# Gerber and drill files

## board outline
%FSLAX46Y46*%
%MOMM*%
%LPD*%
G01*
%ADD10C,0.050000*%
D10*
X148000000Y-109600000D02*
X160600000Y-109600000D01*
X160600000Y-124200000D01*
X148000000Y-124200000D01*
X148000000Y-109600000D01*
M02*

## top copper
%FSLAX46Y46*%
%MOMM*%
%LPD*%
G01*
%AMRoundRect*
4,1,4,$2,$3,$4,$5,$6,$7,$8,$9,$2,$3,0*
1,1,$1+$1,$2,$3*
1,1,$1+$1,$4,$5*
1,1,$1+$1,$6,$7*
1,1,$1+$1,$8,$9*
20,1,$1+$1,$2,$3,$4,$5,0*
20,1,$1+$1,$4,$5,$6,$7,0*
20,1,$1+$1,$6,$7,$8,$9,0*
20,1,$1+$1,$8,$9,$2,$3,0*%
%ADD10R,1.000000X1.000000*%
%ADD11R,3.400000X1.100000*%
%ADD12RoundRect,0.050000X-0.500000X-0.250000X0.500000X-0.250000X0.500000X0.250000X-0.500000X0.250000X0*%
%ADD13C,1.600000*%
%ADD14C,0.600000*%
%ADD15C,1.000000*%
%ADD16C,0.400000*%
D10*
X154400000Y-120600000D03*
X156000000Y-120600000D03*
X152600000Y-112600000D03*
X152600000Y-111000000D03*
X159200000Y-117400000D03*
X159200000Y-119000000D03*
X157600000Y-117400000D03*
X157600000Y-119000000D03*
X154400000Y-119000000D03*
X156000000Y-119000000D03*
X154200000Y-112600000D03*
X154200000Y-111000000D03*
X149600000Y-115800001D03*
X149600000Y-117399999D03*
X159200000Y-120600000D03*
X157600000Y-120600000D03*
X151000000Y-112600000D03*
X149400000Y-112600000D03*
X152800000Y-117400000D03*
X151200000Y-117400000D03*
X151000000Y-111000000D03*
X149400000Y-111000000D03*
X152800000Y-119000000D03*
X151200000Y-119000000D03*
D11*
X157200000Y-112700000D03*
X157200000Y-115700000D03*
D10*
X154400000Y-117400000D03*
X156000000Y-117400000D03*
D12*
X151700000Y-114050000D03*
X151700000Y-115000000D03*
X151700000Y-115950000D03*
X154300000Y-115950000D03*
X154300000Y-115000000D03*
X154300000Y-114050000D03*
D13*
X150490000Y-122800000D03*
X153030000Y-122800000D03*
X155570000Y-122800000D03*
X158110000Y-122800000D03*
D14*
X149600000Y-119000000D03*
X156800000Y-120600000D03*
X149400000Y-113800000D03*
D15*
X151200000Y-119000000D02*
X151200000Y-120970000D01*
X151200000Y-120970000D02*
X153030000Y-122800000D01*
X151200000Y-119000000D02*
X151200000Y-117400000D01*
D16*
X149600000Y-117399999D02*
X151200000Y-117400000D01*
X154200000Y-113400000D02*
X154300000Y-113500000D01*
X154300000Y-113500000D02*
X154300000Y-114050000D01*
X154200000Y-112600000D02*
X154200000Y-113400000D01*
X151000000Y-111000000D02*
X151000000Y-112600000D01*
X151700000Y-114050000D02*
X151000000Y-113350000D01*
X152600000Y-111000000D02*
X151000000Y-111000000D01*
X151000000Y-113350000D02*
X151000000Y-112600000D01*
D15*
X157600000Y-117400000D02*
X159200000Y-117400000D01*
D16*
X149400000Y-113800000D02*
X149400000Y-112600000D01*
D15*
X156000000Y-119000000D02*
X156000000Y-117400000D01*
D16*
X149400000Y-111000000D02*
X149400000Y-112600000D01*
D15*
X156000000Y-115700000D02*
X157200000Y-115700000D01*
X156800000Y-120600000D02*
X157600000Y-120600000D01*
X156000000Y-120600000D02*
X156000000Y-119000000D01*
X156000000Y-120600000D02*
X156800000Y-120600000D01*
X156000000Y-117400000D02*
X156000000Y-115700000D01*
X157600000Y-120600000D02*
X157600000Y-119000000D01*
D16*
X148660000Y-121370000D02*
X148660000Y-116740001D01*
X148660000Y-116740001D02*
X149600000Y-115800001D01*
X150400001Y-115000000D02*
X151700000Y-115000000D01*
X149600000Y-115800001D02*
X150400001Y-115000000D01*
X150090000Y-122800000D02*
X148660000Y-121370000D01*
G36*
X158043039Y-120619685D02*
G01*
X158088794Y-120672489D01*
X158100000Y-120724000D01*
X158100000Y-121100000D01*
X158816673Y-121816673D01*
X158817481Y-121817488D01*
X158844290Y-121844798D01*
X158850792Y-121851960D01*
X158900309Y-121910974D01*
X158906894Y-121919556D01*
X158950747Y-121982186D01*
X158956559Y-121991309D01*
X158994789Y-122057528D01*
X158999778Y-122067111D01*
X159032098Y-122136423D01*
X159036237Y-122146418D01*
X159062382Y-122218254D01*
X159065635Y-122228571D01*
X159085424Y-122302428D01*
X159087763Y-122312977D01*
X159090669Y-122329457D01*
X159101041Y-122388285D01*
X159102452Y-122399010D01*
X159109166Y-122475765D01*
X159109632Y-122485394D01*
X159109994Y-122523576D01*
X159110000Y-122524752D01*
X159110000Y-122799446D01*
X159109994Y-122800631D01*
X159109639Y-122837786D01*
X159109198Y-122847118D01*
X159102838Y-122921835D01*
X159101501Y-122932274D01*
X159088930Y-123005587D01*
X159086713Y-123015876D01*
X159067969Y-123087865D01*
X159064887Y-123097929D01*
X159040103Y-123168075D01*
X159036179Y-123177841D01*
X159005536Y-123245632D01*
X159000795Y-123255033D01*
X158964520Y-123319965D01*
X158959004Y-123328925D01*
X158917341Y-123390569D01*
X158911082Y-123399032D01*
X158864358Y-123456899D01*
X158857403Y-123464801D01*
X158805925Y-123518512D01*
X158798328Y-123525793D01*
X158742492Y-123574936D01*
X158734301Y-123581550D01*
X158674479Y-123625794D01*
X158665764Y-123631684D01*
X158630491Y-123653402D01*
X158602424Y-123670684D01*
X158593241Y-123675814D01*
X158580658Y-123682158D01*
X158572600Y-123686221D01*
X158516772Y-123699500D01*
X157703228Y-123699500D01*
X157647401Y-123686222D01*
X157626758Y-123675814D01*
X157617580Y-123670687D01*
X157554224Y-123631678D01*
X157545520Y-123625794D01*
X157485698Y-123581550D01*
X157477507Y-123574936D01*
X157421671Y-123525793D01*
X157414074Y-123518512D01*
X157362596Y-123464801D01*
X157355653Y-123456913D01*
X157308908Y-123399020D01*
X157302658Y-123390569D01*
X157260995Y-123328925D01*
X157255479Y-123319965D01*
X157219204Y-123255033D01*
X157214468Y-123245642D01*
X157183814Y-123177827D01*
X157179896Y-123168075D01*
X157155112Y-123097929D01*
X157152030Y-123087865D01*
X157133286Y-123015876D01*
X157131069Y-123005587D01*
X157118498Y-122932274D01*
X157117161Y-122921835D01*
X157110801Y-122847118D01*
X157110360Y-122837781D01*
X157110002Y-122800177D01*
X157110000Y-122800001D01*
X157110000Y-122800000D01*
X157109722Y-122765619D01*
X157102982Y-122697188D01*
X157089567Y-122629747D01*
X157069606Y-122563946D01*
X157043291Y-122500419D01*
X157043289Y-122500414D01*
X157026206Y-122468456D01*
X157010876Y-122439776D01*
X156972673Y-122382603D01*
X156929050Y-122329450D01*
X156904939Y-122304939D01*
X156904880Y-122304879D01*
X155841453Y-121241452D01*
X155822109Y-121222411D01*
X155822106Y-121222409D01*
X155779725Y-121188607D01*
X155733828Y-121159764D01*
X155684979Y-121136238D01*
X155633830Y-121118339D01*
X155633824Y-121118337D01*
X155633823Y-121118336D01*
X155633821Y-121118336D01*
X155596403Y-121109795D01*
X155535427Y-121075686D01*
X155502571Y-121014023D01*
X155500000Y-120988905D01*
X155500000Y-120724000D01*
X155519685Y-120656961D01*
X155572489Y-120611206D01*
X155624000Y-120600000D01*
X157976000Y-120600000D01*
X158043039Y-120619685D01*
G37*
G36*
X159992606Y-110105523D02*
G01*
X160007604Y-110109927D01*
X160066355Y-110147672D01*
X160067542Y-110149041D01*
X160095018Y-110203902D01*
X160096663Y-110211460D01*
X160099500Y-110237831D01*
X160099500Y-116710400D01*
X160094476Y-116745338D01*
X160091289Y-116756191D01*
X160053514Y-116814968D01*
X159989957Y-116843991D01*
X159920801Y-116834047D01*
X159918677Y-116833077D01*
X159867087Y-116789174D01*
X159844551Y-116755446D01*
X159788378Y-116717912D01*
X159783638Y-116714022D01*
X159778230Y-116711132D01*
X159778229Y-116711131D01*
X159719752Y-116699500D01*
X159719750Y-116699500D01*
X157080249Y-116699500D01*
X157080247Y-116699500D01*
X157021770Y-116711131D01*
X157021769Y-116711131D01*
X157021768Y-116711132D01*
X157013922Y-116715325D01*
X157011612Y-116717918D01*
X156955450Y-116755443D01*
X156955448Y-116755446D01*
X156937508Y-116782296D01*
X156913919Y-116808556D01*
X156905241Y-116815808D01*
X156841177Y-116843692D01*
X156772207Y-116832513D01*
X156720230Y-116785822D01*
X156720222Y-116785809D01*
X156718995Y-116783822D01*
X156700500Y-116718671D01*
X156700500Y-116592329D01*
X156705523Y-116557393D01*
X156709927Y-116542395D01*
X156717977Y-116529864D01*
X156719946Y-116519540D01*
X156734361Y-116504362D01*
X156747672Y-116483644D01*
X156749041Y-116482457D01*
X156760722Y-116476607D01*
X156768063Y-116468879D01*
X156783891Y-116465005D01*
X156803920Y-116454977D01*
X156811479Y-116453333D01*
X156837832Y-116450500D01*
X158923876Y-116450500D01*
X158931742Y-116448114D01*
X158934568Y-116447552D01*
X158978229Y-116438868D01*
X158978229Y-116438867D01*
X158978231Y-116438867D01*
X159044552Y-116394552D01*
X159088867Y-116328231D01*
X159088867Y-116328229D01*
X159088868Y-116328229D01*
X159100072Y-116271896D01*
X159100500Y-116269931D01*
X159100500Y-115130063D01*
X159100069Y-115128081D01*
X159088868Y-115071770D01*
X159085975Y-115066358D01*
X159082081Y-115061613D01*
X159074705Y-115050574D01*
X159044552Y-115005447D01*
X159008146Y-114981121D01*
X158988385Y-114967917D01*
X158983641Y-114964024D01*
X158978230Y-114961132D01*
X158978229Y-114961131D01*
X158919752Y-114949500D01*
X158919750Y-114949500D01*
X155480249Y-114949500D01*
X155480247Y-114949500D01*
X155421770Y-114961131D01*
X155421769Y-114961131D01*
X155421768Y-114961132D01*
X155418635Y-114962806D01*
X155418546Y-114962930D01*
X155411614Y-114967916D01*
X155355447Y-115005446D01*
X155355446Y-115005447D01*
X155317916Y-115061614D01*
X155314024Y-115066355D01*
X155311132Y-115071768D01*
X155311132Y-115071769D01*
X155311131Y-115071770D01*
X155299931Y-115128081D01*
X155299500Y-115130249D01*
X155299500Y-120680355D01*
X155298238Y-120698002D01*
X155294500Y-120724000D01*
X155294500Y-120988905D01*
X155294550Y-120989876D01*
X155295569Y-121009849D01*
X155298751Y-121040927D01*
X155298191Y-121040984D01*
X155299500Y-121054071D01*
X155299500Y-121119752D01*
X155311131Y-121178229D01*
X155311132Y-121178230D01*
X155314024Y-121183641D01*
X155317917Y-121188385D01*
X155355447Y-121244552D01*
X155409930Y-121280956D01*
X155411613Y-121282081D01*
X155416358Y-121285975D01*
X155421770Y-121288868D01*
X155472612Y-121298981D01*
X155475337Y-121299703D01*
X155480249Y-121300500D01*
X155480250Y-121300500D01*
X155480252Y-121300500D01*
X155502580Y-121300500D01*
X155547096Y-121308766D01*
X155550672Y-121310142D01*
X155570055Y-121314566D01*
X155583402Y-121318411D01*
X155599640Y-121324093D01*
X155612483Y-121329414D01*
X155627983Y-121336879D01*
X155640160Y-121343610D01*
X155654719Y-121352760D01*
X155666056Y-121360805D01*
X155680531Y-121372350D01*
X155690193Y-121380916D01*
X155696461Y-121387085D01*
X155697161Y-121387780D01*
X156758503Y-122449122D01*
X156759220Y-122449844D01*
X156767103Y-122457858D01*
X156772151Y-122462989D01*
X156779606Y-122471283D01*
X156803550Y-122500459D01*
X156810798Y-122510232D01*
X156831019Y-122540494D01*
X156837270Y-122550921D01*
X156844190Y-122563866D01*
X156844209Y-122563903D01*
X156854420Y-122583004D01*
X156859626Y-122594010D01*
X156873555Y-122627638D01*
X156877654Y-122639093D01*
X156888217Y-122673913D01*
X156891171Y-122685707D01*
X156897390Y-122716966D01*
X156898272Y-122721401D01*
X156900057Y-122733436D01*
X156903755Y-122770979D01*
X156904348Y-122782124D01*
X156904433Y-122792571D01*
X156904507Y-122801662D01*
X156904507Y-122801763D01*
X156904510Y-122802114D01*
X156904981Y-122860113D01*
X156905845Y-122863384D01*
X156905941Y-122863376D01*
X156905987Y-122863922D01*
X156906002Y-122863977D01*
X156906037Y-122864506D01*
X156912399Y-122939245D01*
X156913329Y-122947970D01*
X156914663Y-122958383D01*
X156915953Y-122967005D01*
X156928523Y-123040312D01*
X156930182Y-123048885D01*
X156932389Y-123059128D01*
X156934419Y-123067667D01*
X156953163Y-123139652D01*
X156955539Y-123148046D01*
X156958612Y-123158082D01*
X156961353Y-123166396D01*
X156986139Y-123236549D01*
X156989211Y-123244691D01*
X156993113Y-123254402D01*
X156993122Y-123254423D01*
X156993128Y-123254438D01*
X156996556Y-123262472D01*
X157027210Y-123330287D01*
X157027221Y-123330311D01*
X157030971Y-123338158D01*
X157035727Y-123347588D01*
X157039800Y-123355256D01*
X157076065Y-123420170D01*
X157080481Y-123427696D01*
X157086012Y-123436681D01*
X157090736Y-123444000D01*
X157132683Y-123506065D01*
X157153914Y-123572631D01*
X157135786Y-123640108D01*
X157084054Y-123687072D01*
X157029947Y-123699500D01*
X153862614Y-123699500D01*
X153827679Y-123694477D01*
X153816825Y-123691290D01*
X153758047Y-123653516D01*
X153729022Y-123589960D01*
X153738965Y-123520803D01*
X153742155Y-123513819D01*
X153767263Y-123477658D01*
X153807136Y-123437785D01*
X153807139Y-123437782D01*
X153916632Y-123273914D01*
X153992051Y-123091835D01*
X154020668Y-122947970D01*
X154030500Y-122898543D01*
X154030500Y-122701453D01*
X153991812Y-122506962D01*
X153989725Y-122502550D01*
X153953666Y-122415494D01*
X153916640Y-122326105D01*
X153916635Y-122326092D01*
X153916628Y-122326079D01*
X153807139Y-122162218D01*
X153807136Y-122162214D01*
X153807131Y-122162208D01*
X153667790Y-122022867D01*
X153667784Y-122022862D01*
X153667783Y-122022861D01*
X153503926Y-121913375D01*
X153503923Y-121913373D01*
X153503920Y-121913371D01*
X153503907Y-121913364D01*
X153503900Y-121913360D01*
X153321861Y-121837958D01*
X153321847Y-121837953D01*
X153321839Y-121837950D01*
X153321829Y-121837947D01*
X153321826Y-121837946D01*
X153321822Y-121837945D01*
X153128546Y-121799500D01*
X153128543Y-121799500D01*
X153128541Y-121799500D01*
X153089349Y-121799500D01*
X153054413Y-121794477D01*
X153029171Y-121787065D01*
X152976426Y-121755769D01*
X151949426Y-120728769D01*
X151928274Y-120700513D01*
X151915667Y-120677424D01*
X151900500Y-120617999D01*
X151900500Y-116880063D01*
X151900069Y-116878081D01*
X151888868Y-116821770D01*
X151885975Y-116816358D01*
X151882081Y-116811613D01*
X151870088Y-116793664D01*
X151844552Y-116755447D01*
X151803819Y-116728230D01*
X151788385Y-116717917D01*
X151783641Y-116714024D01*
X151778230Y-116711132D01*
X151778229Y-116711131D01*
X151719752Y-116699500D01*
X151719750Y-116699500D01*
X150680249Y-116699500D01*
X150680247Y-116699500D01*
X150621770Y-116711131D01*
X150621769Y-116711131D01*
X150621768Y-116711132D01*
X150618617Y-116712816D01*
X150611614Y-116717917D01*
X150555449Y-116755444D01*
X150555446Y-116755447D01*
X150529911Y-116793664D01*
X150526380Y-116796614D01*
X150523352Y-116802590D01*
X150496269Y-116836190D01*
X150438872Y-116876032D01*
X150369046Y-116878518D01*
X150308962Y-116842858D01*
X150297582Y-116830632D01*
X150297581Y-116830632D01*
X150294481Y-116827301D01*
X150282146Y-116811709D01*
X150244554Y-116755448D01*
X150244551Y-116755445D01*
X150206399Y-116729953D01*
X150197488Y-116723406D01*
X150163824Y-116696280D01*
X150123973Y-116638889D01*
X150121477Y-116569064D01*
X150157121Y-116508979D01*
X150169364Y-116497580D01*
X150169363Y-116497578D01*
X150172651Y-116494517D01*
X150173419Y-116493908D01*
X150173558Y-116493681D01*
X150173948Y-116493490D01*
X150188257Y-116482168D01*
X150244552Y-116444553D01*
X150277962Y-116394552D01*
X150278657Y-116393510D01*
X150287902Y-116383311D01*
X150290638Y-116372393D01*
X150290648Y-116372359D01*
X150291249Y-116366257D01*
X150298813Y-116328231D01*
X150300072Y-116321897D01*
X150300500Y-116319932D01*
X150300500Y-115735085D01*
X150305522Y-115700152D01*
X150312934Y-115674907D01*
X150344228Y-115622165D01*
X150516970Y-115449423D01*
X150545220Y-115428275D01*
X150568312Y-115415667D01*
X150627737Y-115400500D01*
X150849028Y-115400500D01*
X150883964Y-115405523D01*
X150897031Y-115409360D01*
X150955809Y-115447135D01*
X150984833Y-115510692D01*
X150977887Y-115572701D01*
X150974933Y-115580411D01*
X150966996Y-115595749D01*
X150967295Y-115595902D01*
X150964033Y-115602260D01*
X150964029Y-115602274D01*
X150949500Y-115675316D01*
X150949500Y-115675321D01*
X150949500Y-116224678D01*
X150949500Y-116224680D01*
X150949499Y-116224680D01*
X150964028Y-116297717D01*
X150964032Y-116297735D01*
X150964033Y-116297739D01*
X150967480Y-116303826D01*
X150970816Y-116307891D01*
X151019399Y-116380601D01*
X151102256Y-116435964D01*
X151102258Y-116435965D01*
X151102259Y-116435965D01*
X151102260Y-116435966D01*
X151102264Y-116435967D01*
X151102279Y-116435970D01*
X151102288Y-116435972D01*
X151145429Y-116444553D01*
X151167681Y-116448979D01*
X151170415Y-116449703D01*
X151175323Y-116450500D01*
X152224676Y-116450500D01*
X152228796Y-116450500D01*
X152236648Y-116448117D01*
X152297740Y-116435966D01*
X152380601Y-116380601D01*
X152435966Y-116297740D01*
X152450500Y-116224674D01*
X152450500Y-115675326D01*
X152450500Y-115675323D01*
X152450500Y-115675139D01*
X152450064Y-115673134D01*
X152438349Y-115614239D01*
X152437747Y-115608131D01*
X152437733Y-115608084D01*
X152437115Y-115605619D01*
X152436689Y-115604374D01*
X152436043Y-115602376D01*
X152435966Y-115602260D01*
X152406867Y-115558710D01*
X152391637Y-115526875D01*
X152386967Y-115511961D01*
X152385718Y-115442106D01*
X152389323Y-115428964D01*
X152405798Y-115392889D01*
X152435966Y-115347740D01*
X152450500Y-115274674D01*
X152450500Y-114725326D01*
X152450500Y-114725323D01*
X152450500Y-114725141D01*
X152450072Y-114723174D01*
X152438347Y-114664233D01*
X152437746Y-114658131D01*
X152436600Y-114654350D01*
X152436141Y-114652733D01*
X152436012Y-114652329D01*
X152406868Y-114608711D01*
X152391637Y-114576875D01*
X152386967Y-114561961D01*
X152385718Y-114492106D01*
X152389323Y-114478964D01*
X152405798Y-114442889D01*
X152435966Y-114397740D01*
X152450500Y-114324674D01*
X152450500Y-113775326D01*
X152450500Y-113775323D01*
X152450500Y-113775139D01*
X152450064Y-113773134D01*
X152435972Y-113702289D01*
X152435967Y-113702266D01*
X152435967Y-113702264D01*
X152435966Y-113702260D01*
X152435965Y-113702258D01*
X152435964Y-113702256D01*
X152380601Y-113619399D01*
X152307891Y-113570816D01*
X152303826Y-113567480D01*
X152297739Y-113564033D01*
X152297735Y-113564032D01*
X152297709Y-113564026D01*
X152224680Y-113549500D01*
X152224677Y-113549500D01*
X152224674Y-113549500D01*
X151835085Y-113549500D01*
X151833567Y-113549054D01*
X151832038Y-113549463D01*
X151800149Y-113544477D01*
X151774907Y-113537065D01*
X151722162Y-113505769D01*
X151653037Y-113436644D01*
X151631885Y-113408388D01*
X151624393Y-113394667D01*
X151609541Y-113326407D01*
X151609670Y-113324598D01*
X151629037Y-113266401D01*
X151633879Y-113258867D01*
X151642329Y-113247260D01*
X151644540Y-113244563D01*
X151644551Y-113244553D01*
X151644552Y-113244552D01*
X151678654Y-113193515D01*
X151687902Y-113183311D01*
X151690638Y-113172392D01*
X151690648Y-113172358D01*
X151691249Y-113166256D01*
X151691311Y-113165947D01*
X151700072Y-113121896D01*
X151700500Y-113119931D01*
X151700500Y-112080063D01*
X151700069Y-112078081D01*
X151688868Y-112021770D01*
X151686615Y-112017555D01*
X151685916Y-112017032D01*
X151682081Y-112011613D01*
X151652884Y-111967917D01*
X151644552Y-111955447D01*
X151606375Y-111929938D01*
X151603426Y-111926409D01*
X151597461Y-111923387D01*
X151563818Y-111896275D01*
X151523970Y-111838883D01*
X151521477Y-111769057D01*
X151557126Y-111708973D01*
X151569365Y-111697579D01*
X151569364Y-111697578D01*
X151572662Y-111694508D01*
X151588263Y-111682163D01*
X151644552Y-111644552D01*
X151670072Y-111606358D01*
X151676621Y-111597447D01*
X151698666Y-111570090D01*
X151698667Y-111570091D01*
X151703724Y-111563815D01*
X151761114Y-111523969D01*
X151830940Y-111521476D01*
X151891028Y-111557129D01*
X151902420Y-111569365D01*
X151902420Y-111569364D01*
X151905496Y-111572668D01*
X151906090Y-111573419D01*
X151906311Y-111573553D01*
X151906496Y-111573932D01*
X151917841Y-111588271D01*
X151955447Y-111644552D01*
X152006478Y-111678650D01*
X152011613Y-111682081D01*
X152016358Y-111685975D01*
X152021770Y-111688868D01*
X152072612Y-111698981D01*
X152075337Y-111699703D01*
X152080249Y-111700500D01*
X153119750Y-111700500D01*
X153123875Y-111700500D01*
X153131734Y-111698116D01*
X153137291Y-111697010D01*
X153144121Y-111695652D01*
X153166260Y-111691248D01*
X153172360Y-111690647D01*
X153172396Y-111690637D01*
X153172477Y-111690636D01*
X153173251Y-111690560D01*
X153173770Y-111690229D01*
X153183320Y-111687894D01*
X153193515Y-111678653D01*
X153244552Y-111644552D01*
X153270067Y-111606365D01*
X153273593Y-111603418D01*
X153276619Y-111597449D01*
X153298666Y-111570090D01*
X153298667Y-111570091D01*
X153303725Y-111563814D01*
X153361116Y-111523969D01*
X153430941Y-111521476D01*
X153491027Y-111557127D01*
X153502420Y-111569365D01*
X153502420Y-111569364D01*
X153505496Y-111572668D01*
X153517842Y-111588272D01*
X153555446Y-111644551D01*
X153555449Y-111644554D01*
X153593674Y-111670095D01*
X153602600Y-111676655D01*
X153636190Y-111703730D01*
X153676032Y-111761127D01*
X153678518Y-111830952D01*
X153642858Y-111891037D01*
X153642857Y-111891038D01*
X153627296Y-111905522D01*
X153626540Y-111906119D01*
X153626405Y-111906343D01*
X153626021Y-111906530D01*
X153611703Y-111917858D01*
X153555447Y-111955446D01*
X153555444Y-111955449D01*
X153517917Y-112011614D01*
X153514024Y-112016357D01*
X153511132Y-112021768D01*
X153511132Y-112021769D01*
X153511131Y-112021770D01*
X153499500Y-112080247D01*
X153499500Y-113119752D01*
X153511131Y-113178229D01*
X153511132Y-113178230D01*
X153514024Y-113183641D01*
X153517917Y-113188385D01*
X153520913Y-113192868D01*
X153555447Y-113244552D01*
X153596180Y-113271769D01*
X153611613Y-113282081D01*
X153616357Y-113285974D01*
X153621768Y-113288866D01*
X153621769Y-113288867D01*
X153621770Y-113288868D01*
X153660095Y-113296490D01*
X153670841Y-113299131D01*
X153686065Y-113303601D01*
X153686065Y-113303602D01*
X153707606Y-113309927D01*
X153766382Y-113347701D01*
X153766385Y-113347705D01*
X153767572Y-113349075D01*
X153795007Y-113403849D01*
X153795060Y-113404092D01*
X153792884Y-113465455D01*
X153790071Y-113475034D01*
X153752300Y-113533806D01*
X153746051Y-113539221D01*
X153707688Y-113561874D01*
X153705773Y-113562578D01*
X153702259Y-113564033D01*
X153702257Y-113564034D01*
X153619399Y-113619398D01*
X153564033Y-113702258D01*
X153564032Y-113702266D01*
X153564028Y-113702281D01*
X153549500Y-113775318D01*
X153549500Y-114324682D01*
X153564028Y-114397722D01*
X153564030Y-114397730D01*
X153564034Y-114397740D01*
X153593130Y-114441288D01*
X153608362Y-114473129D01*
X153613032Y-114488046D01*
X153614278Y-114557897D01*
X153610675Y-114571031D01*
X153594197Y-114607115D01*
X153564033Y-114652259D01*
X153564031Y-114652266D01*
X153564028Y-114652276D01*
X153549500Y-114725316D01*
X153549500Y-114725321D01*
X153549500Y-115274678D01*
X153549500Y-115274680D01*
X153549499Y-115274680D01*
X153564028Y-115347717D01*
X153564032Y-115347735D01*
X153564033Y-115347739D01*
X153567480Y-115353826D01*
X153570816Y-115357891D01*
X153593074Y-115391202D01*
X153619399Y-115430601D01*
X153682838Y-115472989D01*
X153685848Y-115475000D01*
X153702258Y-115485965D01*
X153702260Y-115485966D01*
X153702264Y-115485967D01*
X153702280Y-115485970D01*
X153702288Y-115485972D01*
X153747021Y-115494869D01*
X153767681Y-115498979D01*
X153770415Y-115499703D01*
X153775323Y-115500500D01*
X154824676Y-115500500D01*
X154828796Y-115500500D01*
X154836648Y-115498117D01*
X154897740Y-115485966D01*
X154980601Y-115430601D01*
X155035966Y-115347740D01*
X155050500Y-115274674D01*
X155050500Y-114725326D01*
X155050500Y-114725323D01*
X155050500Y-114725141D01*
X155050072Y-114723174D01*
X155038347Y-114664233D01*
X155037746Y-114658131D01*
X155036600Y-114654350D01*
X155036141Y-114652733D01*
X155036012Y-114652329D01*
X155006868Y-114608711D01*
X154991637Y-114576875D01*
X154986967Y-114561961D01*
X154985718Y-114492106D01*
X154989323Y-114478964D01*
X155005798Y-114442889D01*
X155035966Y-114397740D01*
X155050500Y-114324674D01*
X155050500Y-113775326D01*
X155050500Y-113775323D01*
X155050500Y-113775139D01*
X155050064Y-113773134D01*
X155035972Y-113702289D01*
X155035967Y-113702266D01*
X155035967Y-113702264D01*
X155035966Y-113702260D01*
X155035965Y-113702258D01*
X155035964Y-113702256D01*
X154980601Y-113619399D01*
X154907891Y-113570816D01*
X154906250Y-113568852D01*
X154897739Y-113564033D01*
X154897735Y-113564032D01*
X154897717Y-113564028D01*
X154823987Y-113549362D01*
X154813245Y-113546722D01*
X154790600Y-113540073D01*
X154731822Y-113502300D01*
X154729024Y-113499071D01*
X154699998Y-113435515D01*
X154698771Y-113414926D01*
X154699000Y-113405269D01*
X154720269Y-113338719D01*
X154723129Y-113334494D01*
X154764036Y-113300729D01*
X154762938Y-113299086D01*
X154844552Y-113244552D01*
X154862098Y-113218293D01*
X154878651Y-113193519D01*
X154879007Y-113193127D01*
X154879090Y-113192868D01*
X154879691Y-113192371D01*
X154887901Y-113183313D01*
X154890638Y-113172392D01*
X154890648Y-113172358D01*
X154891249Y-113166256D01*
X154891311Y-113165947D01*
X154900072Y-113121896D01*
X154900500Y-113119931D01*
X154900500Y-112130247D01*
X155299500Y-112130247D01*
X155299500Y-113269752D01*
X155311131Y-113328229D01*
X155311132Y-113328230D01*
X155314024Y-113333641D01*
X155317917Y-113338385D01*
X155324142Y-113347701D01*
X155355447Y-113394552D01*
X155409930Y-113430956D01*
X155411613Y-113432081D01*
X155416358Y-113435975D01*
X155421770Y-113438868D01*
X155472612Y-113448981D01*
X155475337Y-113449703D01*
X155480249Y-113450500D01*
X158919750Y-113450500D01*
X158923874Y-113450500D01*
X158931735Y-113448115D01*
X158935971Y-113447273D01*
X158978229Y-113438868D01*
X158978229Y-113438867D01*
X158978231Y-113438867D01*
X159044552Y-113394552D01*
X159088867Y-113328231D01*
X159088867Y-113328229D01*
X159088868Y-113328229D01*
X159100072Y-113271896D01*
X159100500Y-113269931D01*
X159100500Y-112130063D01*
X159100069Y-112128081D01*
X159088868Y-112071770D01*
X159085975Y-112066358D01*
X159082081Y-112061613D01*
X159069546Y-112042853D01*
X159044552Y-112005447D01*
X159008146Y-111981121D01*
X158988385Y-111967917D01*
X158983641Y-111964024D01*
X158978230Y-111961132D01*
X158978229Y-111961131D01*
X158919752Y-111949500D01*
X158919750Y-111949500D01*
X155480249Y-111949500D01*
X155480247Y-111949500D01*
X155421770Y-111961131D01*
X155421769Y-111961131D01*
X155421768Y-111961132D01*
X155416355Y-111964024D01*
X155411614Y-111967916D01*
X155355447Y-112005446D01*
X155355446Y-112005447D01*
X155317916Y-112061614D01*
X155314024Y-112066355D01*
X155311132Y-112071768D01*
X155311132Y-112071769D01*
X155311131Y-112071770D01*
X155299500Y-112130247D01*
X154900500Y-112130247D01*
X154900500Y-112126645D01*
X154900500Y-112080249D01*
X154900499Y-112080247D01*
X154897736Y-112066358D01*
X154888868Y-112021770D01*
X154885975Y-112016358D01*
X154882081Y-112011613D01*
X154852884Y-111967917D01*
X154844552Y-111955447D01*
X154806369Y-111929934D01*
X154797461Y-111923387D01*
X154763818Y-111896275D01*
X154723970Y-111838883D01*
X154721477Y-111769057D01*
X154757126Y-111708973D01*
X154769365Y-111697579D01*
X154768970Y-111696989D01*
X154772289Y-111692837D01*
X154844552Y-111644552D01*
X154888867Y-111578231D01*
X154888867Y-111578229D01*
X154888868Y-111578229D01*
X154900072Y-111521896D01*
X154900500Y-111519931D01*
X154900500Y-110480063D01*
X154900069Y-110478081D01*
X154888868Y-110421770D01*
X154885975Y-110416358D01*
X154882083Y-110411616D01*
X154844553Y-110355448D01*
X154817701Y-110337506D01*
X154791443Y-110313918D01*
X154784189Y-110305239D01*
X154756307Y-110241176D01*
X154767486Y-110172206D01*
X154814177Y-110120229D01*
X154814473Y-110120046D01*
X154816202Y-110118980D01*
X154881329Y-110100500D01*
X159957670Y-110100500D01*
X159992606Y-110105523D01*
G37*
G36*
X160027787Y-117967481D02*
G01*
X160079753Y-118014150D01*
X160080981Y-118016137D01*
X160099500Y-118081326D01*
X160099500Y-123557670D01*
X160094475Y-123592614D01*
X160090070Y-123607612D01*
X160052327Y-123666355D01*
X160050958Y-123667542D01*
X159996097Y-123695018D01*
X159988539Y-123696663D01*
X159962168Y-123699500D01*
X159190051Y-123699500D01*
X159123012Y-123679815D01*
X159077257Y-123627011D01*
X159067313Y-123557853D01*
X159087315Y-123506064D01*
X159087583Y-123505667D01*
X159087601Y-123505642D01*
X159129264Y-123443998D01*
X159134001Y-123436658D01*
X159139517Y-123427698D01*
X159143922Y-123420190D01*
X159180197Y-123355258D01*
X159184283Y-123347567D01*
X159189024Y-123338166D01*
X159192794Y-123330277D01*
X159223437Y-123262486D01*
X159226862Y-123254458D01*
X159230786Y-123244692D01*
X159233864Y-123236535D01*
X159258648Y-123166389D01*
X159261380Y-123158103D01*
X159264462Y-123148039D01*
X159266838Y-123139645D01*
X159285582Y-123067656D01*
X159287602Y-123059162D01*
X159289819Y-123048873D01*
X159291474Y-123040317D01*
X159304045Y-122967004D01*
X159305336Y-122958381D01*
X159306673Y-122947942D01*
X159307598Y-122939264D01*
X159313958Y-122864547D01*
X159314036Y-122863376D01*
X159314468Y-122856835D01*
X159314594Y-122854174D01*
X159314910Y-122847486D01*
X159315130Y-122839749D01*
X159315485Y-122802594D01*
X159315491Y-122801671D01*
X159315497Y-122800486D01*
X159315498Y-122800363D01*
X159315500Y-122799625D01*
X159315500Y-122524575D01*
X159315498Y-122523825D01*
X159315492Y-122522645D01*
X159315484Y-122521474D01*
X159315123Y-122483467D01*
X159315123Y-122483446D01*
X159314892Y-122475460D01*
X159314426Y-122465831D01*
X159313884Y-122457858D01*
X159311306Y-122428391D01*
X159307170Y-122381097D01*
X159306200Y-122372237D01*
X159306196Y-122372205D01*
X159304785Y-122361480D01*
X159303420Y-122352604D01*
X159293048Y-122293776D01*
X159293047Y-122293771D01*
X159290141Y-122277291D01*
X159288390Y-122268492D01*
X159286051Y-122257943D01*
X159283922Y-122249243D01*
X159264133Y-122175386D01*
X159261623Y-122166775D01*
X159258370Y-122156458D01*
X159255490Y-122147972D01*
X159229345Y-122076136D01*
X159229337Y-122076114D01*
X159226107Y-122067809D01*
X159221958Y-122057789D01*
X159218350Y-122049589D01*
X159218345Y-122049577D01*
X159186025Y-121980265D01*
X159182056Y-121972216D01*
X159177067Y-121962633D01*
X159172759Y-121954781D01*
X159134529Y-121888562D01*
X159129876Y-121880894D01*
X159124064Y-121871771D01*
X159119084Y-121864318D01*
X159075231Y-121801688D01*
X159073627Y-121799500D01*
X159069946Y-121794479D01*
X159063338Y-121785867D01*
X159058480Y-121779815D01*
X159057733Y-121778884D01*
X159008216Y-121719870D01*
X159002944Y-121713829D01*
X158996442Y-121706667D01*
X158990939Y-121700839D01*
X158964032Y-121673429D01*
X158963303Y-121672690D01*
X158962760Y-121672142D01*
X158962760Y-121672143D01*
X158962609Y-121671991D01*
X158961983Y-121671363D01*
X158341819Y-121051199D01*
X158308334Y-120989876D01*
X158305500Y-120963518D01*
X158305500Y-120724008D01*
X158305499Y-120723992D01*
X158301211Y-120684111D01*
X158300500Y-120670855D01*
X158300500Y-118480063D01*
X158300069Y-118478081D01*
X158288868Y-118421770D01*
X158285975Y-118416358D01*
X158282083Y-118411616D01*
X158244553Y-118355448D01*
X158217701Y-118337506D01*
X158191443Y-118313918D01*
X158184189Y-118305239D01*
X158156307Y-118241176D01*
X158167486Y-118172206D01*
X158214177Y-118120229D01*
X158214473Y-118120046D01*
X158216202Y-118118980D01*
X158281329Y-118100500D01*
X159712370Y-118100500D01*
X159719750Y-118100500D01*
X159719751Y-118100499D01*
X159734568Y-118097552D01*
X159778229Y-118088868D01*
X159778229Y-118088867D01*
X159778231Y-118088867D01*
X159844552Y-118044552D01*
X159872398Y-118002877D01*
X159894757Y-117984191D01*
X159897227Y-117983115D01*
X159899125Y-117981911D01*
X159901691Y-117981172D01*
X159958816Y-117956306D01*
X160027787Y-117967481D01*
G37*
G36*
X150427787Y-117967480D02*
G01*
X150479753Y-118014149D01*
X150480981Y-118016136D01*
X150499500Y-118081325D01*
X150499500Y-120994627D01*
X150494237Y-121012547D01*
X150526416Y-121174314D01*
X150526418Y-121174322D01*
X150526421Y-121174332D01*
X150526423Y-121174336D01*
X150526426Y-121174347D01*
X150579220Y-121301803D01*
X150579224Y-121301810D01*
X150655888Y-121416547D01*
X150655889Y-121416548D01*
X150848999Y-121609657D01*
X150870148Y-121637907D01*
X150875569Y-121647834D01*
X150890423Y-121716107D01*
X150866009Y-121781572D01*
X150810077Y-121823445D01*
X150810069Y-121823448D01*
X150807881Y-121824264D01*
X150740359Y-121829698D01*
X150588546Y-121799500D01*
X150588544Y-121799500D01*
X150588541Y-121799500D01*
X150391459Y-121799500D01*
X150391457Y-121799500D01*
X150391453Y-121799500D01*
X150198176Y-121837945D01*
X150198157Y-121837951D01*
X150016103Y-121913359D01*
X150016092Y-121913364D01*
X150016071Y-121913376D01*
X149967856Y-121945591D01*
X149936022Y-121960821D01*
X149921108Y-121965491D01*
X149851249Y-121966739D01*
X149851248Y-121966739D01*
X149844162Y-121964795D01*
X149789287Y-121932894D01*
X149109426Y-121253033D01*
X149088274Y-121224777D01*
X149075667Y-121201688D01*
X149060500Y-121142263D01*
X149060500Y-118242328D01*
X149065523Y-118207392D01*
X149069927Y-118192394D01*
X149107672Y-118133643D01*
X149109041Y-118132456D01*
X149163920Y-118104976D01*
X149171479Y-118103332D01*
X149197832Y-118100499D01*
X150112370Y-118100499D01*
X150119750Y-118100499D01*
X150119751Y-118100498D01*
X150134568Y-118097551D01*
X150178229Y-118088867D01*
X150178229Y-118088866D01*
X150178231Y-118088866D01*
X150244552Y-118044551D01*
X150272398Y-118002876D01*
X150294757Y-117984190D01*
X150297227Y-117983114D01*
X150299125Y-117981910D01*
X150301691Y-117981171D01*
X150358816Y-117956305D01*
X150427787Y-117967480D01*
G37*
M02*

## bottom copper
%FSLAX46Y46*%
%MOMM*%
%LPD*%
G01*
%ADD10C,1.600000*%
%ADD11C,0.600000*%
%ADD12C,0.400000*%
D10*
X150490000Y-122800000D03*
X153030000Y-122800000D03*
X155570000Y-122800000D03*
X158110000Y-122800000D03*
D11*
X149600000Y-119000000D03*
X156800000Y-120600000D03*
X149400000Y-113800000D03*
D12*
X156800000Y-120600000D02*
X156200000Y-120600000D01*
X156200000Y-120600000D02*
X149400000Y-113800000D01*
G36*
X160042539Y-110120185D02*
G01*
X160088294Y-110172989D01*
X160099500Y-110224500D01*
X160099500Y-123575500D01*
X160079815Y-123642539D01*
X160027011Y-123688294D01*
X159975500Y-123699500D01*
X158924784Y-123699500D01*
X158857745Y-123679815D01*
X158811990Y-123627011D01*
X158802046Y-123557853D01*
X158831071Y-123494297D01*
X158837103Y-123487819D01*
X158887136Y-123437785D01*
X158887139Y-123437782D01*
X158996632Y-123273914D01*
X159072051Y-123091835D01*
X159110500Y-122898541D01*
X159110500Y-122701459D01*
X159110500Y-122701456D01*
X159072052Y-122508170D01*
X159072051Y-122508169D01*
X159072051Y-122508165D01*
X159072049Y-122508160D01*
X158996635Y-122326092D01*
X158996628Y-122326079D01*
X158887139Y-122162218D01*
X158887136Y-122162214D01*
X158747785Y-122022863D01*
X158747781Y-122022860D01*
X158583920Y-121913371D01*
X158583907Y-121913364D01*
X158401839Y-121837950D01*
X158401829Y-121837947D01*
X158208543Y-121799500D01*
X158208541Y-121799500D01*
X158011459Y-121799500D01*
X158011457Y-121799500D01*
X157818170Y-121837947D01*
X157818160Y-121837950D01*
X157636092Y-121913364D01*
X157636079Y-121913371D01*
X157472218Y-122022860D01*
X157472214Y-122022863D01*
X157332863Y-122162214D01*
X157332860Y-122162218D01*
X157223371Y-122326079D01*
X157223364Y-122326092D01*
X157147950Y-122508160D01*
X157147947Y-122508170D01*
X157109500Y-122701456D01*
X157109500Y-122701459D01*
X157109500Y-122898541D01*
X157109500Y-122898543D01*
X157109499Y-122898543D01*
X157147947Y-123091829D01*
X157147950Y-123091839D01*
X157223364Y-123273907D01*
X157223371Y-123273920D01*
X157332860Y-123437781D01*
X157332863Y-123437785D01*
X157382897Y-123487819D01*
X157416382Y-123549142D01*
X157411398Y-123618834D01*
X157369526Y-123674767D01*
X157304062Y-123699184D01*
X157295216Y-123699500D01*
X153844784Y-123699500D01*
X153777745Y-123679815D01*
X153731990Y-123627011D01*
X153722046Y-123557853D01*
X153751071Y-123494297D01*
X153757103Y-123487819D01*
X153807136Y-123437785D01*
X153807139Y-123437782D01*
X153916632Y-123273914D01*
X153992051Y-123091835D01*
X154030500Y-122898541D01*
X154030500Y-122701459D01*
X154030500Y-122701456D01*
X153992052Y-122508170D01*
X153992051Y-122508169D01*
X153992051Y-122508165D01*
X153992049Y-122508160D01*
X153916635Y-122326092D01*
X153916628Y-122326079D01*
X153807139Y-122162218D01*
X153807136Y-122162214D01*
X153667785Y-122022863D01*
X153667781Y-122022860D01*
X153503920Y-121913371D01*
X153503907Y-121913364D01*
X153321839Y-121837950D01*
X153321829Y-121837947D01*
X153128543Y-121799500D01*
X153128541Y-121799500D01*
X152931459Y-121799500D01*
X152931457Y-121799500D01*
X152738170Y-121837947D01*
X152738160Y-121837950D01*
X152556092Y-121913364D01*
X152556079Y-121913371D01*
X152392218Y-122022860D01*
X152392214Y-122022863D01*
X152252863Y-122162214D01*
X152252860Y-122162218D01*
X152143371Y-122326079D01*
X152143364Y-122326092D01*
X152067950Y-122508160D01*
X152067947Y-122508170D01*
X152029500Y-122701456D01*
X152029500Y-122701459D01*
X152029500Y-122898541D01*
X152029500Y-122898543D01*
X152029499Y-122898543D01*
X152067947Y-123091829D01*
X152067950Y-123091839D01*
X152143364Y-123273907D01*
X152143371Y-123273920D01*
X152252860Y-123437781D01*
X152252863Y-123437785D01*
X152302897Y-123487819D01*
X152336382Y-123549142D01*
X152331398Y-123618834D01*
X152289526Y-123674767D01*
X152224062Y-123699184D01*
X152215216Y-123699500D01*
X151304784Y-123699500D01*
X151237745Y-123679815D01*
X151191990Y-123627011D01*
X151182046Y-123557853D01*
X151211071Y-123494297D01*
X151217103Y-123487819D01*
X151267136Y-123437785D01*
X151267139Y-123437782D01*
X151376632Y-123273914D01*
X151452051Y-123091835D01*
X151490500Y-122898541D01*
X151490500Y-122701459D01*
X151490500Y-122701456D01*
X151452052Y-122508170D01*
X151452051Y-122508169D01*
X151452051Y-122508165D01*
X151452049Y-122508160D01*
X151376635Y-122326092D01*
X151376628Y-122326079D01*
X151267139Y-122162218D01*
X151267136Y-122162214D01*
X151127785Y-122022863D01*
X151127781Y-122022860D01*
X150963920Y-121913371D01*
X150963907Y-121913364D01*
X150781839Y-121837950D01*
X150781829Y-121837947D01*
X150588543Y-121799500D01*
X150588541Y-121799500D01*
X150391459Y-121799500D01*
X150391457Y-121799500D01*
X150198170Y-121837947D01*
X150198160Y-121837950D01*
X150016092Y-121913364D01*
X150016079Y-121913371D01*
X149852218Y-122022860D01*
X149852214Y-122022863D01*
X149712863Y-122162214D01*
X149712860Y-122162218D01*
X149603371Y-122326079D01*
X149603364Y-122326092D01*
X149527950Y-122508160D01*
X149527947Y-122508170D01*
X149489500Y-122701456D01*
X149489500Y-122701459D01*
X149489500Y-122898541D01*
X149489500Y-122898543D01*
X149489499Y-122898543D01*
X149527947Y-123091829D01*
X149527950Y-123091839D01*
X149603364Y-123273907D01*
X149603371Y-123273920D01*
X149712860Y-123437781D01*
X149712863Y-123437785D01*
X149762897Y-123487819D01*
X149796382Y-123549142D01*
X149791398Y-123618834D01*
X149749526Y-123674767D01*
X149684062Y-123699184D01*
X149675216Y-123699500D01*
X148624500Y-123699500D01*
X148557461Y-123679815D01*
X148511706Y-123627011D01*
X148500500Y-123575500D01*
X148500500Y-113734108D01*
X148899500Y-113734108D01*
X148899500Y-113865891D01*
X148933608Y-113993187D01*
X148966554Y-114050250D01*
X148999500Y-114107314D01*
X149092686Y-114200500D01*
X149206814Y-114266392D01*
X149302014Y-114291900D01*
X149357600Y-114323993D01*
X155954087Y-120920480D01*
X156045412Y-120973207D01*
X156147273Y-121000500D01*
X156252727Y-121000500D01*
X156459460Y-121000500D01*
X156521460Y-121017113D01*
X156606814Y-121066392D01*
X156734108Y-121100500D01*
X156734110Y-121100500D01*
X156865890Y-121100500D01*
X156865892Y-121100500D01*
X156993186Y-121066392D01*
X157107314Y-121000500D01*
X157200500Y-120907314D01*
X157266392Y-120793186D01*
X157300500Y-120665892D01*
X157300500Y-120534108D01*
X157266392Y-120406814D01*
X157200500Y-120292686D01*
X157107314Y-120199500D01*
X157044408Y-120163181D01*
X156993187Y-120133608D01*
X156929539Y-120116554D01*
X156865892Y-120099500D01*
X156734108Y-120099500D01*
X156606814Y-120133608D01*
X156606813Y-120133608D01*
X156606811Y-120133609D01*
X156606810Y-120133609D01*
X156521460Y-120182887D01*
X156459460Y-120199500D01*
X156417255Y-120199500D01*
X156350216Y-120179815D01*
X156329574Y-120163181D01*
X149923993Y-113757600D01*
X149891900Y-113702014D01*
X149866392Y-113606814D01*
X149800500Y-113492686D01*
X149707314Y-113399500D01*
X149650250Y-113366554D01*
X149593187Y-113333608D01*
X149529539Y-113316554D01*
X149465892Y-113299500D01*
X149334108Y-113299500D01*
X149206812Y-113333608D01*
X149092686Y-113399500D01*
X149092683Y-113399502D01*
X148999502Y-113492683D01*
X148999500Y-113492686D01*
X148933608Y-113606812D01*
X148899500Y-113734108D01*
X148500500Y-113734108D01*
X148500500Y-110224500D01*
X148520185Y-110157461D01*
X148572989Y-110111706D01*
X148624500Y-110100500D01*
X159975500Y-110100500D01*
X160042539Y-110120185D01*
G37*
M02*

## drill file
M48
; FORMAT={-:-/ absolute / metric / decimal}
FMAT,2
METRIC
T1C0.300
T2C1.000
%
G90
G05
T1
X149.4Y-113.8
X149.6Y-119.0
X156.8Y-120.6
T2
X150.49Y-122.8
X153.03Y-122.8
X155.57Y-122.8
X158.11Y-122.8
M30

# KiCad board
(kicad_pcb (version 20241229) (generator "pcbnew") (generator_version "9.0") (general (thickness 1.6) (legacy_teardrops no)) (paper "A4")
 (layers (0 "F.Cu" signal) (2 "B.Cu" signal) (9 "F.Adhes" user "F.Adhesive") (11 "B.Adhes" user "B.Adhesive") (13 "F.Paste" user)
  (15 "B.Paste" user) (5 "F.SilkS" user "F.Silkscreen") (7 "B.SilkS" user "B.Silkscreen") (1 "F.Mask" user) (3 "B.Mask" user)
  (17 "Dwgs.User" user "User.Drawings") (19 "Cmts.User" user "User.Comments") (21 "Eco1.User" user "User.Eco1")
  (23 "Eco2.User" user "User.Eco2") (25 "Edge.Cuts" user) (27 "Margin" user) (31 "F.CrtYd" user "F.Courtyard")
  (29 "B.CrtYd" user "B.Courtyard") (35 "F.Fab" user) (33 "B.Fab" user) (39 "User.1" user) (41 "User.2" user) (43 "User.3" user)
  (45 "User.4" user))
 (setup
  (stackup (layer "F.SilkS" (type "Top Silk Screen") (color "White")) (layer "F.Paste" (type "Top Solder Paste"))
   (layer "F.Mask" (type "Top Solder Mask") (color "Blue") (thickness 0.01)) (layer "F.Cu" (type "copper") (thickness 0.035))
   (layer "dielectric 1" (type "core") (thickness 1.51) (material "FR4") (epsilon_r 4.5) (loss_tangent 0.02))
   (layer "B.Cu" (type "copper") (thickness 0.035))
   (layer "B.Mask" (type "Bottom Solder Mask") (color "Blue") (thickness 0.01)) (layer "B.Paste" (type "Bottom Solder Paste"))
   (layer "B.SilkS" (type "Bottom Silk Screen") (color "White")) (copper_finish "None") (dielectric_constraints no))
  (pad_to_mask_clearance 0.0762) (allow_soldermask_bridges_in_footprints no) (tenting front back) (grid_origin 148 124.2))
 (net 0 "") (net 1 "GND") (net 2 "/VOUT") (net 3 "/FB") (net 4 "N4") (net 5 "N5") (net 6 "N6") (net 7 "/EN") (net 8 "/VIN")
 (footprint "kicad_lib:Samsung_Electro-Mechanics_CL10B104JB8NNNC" (layer "F.Cu") (at 155.2 120.6)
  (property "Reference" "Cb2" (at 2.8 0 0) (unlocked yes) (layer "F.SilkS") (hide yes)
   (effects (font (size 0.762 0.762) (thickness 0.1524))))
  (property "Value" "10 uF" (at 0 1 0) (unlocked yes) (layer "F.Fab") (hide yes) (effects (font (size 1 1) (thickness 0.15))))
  (pad "1" smd rect (at -0.8 0) (size 1 1) (layers "F.Cu" "F.Mask" "F.Paste") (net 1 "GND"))
  (pad "2" smd rect (at 0.8 0) (size 1 1) (layers "F.Cu" "F.Mask" "F.Paste") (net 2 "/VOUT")))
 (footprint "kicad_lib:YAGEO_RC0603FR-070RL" (layer "F.Cu") (at 152.6 111.8 90)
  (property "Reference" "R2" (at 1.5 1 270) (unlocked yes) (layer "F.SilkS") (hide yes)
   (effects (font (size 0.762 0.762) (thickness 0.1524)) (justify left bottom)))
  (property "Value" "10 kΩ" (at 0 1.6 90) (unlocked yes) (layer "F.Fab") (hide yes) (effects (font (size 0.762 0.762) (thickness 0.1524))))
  (pad "1" smd rect (at -0.8 0 90) (size 1 1) (layers "F.Cu" "F.Mask" "F.Paste") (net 1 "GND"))
  (pad "2" smd rect (at 0.8 0 90) (size 1 1) (layers "F.Cu" "F.Mask" "F.Paste") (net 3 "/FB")))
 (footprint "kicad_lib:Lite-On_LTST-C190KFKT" (layer "F.Cu") (at 159.2 118.2 -90)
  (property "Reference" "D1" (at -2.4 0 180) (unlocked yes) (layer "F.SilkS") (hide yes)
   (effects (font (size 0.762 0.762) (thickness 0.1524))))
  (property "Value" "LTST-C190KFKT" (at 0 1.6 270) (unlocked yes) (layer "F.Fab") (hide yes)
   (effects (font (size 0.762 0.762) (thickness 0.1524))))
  (pad "A" smd rect (at -0.8 0 270) (size 1 1) (layers "F.Cu" "F.Mask" "F.Paste") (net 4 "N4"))
  (pad "K" smd rect (at 0.8 0 270) (size 1 1) (layers "F.Cu" "F.Mask" "F.Paste") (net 1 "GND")))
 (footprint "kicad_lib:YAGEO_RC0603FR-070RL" (layer "F.Cu") (at 157.6 118.2 -90)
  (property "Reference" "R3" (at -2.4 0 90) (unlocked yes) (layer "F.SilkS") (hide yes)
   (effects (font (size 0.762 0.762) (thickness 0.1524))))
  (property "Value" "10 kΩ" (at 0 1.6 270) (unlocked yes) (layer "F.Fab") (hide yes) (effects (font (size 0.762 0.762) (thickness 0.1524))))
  (pad "1" smd rect (at -0.8 0 270) (size 1 1) (layers "F.Cu" "F.Mask" "F.Paste") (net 4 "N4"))
  (pad "2" smd rect (at 0.8 0 270) (size 1 1) (layers "F.Cu" "F.Mask" "F.Paste") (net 2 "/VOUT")))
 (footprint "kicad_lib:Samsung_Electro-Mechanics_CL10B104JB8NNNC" (layer "F.Cu") (at 155.2 119)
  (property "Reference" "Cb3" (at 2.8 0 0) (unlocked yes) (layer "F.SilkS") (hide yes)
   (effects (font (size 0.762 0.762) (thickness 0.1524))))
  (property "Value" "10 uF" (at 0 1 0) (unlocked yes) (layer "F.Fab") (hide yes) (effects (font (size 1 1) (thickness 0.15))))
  (pad "1" smd rect (at -0.8 0) (size 1 1) (layers "F.Cu" "F.Mask" "F.Paste") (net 1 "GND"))
  (pad "2" smd rect (at 0.8 0) (size 1 1) (layers "F.Cu" "F.Mask" "F.Paste") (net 2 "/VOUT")))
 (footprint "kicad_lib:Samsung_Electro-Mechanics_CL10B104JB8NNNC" (layer "F.Cu") (at 154.2 111.8 90)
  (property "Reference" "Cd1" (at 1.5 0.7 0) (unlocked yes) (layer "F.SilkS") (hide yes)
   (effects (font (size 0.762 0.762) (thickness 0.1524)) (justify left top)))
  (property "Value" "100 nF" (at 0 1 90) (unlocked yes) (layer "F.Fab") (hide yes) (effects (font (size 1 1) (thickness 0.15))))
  (pad "1" smd rect (at -0.8 0 90) (size 1 1) (layers "F.Cu" "F.Mask" "F.Paste") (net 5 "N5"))
  (pad "2" smd rect (at 0.8 0 90) (size 1 1) (layers "F.Cu" "F.Mask" "F.Paste") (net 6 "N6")))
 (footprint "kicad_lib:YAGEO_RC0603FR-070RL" (layer "F.Cu") (at 149.6 116.6 -90)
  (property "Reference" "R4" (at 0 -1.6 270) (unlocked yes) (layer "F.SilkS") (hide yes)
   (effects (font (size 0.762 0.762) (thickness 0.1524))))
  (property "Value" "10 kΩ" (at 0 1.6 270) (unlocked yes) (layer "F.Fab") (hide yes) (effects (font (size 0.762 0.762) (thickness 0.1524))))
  (pad "1" smd rect (at -0.799999 0 270) (size 1 1) (layers "F.Cu" "F.Mask" "F.Paste") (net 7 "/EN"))
  (pad "2" smd rect (at 0.799999 0 270) (size 1 1) (layers "F.Cu" "F.Mask" "F.Paste") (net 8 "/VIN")))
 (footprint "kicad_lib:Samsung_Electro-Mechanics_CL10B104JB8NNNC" (layer "F.Cu") (at 158.4 120.6 180)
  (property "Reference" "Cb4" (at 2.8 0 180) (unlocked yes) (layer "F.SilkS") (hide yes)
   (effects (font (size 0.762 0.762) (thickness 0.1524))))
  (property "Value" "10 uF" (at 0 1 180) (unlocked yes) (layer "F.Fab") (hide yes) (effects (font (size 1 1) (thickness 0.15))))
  (pad "1" smd rect (at -0.8 0 180) (size 1 1) (layers "F.Cu" "F.Mask" "F.Paste") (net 1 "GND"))
  (pad "2" smd rect (at 0.8 0 180) (size 1 1) (layers "F.Cu" "F.Mask" "F.Paste") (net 2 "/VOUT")))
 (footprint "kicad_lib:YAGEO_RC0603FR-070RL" (layer "F.Cu") (at 150.2 112.6 180)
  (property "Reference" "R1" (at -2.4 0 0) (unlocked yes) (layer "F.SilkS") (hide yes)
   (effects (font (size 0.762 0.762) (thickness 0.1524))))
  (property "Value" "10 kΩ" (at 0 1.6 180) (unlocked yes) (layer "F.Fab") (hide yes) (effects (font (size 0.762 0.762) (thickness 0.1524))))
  (pad "1" smd rect (at -0.8 0 180) (size 1 1) (layers "F.Cu" "F.Mask" "F.Paste") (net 3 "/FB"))
  (pad "2" smd rect (at 0.8 0 180) (size 1 1) (layers "F.Cu" "F.Mask" "F.Paste") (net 2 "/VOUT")))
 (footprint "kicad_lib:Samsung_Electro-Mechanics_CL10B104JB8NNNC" (layer "F.Cu") (at 152 117.4 180)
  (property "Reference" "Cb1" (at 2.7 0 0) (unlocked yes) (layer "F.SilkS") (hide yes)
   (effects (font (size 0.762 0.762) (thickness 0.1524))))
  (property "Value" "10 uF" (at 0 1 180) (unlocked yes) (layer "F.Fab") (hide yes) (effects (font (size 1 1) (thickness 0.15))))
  (pad "1" smd rect (at -0.8 0 180) (size 1 1) (layers "F.Cu" "F.Mask" "F.Paste") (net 1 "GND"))
  (pad "2" smd rect (at 0.8 0 180) (size 1 1) (layers "F.Cu" "F.Mask" "F.Paste") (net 8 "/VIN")))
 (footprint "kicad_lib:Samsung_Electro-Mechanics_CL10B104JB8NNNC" (layer "F.Cu") (at 150.2 111 180)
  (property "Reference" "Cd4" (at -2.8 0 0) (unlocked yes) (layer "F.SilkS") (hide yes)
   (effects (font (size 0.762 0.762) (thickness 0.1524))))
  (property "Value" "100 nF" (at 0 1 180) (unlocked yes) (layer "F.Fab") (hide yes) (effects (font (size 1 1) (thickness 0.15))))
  (pad "1" smd rect (at -0.8 0 180) (size 1 1) (layers "F.Cu" "F.Mask" "F.Paste") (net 3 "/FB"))
  (pad "2" smd rect (at 0.8 0 180) (size 1 1) (layers "F.Cu" "F.Mask" "F.Paste") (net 2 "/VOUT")))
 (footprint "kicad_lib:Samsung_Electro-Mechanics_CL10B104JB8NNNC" (layer "F.Cu") (at 152 119 180)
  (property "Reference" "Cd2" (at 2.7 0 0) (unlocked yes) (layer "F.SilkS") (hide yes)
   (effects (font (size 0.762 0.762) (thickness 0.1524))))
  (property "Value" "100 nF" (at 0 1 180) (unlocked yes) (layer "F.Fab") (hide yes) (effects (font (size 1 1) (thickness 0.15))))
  (pad "1" smd rect (at -0.8 0 180) (size 1 1) (layers "F.Cu" "F.Mask" "F.Paste") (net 1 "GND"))
  (pad "2" smd rect (at 0.8 0 180) (size 1 1) (layers "F.Cu" "F.Mask" "F.Paste") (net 8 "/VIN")))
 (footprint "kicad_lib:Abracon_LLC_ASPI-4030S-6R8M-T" (layer "F.Cu") (at 157.2 114.2)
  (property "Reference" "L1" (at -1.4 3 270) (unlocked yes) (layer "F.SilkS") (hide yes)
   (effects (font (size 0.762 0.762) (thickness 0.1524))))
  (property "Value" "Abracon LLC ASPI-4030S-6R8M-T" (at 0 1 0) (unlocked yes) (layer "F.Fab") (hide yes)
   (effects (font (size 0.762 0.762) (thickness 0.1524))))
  (pad "1" smd rect (at 0 -1.5 270) (size 1.1 3.4) (layers "F.Cu" "F.Mask" "F.Paste") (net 6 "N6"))
  (pad "2" smd rect (at 0 1.5 270) (size 1.1 3.4) (layers "F.Cu" "F.Mask" "F.Paste") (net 2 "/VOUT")))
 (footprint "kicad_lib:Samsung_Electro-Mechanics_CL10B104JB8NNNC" (layer "F.Cu") (at 155.2 117.4)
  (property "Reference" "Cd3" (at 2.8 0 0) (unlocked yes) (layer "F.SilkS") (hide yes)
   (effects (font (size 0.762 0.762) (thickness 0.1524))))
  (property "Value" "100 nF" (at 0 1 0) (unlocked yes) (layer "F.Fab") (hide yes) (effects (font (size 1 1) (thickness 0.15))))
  (pad "1" smd rect (at -0.8 0) (size 1 1) (layers "F.Cu" "F.Mask" "F.Paste") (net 1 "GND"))
  (pad "2" smd rect (at 0.8 0) (size 1 1) (layers "F.Cu" "F.Mask" "F.Paste") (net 2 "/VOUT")))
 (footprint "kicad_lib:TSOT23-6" (layer "F.Cu") (at 153 115)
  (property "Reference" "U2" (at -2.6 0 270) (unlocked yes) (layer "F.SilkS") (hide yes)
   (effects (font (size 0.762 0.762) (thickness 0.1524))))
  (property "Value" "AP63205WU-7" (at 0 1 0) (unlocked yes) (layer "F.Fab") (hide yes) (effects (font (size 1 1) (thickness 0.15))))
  (pad "1" smd roundrect (at -1.3 -0.95) (size 1.1 0.6) (layers "F.Cu" "F.Mask" "F.Paste") (roundrect_rratio 0.08333333333) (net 3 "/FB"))
  (pad "2" smd roundrect (at -1.3 0) (size 1.1 0.6) (layers "F.Cu" "F.Mask" "F.Paste") (roundrect_rratio 0.08333333333) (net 7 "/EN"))
  (pad "3" smd roundrect (at -1.3 0.95) (size 1.1 0.6) (layers "F.Cu" "F.Mask" "F.Paste") (roundrect_rratio 0.08333333333) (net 8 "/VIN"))
  (pad "4" smd roundrect (at 1.3 0.95) (size 1.1 0.6) (layers "F.Cu" "F.Mask" "F.Paste") (roundrect_rratio 0.08333333333) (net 1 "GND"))
  (pad "5" smd roundrect (at 1.3 0) (size 1.1 0.6) (layers "F.Cu" "F.Mask" "F.Paste") (roundrect_rratio 0.08333333333) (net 6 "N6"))
  (pad "6" smd roundrect (at 1.3 -0.95) (size 1.1 0.6) (layers "F.Cu" "F.Mask" "F.Paste") (roundrect_rratio 0.08333333333) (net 5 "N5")))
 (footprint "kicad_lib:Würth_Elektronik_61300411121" (layer "B.Cu") (at 154.3 122.8)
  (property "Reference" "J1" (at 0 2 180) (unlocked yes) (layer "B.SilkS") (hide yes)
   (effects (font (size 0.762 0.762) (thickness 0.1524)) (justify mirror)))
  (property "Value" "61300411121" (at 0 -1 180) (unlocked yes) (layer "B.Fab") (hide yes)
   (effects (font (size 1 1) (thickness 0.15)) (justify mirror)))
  (pad "1" thru_hole circle (at -3.81 0) (size 1.6 1.6) (drill 1) (layers "*.Cu" "*.Mask") (remove_unused_layers no) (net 7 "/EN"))
  (pad "2" thru_hole circle (at -1.27 0) (size 1.6 1.6) (drill 1) (layers "*.Cu" "*.Mask") (remove_unused_layers no) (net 8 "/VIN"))
  (pad "3" thru_hole circle (at 1.27 0) (size 1.6 1.6) (drill 1) (layers "*.Cu" "*.Mask") (remove_unused_layers no) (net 1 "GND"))
  (pad "4" thru_hole circle (at 3.81 0) (size 1.6 1.6) (drill 1) (layers "*.Cu" "*.Mask") (remove_unused_layers no) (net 2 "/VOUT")))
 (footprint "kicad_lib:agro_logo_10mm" (layer "B.Cu") (at 155.4 114.6 180)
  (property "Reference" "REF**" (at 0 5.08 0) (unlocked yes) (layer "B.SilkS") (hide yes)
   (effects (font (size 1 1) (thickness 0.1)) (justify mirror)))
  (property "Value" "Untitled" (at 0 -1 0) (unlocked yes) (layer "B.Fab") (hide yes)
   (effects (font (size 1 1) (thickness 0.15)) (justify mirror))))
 (gr_rect (start 148 109.6) (end 160.6 124.2) (stroke (width 0.05) (type default)) (fill no) (layer "Edge.Cuts"))
 (segment (start 151.2 119) (end 151.2 120.97) (width 1) (layer "F.Cu") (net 8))
 (segment (start 151.2 120.97) (end 153.03 122.8) (width 1) (layer "F.Cu") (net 8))
 (segment (start 151.2 119) (end 151.2 117.4) (width 1) (layer "F.Cu") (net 8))
 (segment (start 149.6 117.399999) (end 151.2 117.4) (width 0.4) (layer "F.Cu") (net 8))
 (via (at 149.6 119) (size 0.6) (drill 0.3) (layers "F.Cu" "B.Cu") (free yes) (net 1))
 (segment (start 154.2 113.4) (end 154.3 113.5) (width 0.4) (layer "F.Cu") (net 5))
 (segment (start 154.3 113.5) (end 154.3 114.05) (width 0.4) (layer "F.Cu") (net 5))
 (segment (start 154.2 112.6) (end 154.2 113.4) (width 0.4) (layer "F.Cu") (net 5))
 (segment (start 151 111) (end 151 112.6) (width 0.4) (layer "F.Cu") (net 3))
 (segment (start 151.7 114.05) (end 151 113.35) (width 0.4) (layer "F.Cu") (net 3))
 (segment (start 152.6 111) (end 151 111) (width 0.4) (layer "F.Cu") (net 3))
 (segment (start 151 113.35) (end 151 112.6) (width 0.4) (layer "F.Cu") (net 3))
 (segment (start 157.6 117.4) (end 159.2 117.4) (width 1) (layer "F.Cu") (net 4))
 (segment (start 149.4 113.8) (end 149.4 112.6) (width 0.4) (layer "F.Cu") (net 2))
 (segment (start 156 119) (end 156 117.4) (width 1) (layer "F.Cu") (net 2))
 (segment (start 149.4 111) (end 149.4 112.6) (width 0.4) (layer "F.Cu") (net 2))
 (segment (start 156 115.7) (end 157.2 115.7) (width 1) (layer "F.Cu") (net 2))
 (segment (start 156.8 120.6) (end 157.6 120.6) (width 1) (layer "F.Cu") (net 2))
 (segment (start 156 120.6) (end 156 119) (width 1) (layer "F.Cu") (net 2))
 (segment (start 156 120.6) (end 156.8 120.6) (width 1) (layer "F.Cu") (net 2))
 (segment (start 156 117.4) (end 156 115.7) (width 1) (layer "F.Cu") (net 2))
 (segment (start 157.6 120.6) (end 157.6 119) (width 1) (layer "F.Cu") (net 2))
 (via (at 156.8 120.6) (size 0.6) (drill 0.3) (layers "F.Cu" "B.Cu") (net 2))
 (via (at 149.4 113.8) (size 0.6) (drill 0.3) (layers "F.Cu" "B.Cu") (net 2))
 (segment (start 156.8 120.6) (end 156.2 120.6) (width 0.4) (layer "B.Cu") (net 2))
 (segment (start 156.2 120.6) (end 149.4 113.8) (width 0.4) (layer "B.Cu") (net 2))
 (segment (start 148.66 121.37) (end 148.66 116.740001) (width 0.4) (layer "F.Cu") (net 7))
 (segment (start 148.66 116.740001) (end 149.6 115.800001) (width 0.4) (layer "F.Cu") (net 7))
 (segment (start 150.400001 115) (end 151.7 115) (width 0.4) (layer "F.Cu") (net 7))
 (segment (start 149.6 115.800001) (end 150.400001 115) (width 0.4) (layer "F.Cu") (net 7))
 (segment (start 150.09 122.8) (end 148.66 121.37) (width 0.4) (layer "F.Cu") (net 7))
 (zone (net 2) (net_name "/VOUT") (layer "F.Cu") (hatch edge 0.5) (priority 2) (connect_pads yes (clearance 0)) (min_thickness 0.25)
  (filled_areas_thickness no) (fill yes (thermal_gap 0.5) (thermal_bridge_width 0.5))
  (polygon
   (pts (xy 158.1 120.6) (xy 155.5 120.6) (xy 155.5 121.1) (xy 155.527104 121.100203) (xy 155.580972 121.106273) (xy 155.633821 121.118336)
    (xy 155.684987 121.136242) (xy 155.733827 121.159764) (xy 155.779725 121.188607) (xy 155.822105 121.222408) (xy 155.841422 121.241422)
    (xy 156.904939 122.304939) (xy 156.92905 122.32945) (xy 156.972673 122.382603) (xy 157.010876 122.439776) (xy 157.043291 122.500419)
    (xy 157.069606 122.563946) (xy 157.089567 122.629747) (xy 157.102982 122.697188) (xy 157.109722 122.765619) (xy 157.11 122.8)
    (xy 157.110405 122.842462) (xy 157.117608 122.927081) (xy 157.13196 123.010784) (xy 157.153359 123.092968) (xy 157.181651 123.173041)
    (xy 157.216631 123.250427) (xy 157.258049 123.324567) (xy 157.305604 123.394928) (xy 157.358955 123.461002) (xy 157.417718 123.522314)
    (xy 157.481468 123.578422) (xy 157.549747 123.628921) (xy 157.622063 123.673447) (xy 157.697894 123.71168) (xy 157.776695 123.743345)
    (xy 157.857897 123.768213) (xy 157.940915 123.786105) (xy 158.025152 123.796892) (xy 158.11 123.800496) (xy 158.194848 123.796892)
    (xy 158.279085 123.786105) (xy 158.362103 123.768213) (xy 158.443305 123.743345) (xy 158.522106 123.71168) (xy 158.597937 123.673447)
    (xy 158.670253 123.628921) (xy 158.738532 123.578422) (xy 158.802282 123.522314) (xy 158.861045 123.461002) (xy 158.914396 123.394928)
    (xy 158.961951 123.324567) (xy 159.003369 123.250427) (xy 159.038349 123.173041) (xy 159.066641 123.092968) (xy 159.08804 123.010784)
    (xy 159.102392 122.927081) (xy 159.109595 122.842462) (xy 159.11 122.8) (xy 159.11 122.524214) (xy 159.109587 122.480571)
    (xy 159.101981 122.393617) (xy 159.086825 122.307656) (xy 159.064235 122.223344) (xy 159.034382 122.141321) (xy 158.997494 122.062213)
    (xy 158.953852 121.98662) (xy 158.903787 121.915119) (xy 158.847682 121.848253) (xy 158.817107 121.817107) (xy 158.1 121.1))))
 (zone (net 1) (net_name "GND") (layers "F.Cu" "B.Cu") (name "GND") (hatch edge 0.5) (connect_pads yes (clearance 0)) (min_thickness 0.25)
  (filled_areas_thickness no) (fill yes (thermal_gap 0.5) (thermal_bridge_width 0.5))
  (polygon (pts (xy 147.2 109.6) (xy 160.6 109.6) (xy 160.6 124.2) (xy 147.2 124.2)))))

